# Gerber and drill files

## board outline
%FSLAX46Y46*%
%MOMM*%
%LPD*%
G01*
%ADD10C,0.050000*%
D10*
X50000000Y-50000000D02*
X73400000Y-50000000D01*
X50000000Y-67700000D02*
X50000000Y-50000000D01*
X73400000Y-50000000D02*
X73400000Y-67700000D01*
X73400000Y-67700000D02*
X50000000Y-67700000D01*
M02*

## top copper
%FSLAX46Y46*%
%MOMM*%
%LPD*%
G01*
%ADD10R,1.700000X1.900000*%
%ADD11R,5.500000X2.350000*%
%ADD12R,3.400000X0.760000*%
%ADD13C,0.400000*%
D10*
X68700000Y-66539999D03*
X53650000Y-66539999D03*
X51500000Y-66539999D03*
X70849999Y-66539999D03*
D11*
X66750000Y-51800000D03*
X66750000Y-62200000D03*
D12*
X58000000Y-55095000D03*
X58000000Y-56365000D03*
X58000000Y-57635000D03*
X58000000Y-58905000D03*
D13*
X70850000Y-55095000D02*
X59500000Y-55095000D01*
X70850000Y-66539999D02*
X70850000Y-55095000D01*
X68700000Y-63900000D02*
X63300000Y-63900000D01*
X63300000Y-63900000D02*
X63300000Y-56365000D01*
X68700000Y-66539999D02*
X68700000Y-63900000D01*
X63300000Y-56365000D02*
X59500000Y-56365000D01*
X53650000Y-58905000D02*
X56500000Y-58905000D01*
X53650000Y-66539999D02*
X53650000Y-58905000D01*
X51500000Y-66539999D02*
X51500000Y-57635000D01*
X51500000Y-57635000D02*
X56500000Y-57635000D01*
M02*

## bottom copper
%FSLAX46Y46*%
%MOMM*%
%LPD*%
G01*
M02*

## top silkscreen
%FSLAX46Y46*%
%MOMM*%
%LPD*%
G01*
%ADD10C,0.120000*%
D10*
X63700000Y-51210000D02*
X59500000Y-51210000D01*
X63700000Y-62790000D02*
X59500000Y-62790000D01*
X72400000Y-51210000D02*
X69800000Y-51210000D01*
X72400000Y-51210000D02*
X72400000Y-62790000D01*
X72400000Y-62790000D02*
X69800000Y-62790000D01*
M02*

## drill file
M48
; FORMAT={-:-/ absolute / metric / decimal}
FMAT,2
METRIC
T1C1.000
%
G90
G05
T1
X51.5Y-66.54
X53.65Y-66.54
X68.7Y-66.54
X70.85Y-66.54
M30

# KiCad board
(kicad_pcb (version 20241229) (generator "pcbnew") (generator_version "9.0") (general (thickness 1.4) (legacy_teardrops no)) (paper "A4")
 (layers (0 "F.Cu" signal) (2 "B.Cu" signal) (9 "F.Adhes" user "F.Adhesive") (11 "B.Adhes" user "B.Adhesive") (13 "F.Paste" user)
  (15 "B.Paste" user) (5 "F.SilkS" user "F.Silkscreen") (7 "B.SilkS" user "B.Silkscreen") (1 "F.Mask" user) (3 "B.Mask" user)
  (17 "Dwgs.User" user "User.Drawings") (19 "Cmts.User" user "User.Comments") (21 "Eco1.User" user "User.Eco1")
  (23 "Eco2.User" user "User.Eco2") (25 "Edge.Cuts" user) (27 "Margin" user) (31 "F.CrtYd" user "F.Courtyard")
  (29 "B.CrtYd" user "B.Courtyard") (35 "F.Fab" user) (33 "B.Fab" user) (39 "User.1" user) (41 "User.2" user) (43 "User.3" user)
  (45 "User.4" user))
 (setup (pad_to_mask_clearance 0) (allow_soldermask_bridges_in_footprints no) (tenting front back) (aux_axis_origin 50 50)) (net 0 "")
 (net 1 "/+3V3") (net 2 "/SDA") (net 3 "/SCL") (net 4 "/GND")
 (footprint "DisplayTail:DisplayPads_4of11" (layer "F.Cu") (at 51.5 66.539999)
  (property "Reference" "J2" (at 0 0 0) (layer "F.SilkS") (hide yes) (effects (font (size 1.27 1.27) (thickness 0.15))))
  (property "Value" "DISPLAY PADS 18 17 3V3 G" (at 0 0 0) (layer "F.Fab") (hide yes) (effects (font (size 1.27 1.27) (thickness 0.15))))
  (pad "3V3" thru_hole rect (at 17.2 0) (size 1.7 1.9) (drill 1) (layers "*.Cu" "*.Mask") (remove_unused_layers yes) (keep_end_layers no)
   (zone_layer_connections) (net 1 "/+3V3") (thermal_bridge_angle 45))
  (pad "17" thru_hole rect (at 2.15 0) (size 1.7 1.9) (drill 1) (layers "*.Cu" "*.Mask") (remove_unused_layers yes) (keep_end_layers no)
   (zone_layer_connections) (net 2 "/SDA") (thermal_bridge_angle 45))
  (pad "18" thru_hole rect (at 0 0) (size 1.7 1.9) (drill 1) (layers "*.Cu" "*.Mask") (remove_unused_layers yes) (keep_end_layers no)
   (zone_layer_connections) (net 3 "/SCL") (thermal_bridge_angle 45))
  (pad "G" thru_hole rect (at 19.349999 0) (size 1.7 1.9) (drill 1) (layers "*.Cu" "*.Mask") (remove_unused_layers yes) (keep_end_layers no)
   (zone_layer_connections) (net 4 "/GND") (thermal_bridge_angle 45)))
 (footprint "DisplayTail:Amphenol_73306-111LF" (layer "F.Cu") (at 72.4 57 -90)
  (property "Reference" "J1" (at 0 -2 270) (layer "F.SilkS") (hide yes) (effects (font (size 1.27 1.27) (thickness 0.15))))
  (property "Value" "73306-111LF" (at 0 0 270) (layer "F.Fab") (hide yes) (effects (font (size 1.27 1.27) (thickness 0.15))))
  (fp_line (start -5.79 8.7) (end -5.79 12.9) (stroke (width 0.12) (type default)) (layer "F.SilkS"))
  (fp_line (start 5.79 8.7) (end 5.79 12.9) (stroke (width 0.12) (type default)) (layer "F.SilkS"))
  (fp_line (start -5.79 0) (end -5.79 2.6) (stroke (width 0.12) (type default)) (layer "F.SilkS"))
  (fp_line (start -5.79 0) (end 5.79 0) (stroke (width 0.12) (type default)) (layer "F.SilkS"))
  (fp_line (start 5.79 0) (end 5.79 2.6) (stroke (width 0.12) (type default)) (layer "F.SilkS"))
  (pad "" smd rect (at -5.2 5.65 270) (size 2.35 5.5) (layers "F.Cu" "F.Mask" "F.Paste") (thermal_bridge_angle 45))
  (pad "" smd rect (at 5.2 5.65 270) (size 2.35 5.5) (layers "F.Cu" "F.Mask" "F.Paste") (thermal_bridge_angle 45))
  (pad "1" smd rect (at -1.905 14.4 270) (size 0.76 3.4) (layers "F.Cu" "F.Mask" "F.Paste") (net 4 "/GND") (thermal_bridge_angle 45))
  (pad "2" smd rect (at -0.635 14.4 270) (size 0.76 3.4) (layers "F.Cu" "F.Mask" "F.Paste") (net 1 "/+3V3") (thermal_bridge_angle 45))
  (pad "3" smd rect (at 0.635 14.4 270) (size 0.76 3.4) (layers "F.Cu" "F.Mask" "F.Paste") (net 3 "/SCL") (thermal_bridge_angle 45))
  (pad "4" smd rect (at 1.905 14.4 270) (size 0.76 3.4) (layers "F.Cu" "F.Mask" "F.Paste") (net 2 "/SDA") (thermal_bridge_angle 45)))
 (gr_line (start 50 50) (end 73.4 50) (stroke (width 0.05) (type default)) (layer "Edge.Cuts"))
 (gr_line (start 50 67.7) (end 50 50) (stroke (width 0.05) (type default)) (layer "Edge.Cuts"))
 (gr_line (start 73.4 50) (end 73.4 67.7) (stroke (width 0.05) (type default)) (layer "Edge.Cuts"))
 (gr_line (start 73.4 67.7) (end 50 67.7) (stroke (width 0.05) (type default)) (layer "Edge.Cuts"))
 (segment (start 70.85 55.095) (end 59.5 55.095) (width 0.4) (layer "F.Cu") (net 4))
 (segment (start 70.85 66.539999) (end 70.85 55.095) (width 0.4) (layer "F.Cu") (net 4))
 (segment (start 68.7 63.9) (end 63.3 63.9) (width 0.4) (layer "F.Cu") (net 1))
 (segment (start 63.3 63.9) (end 63.3 56.365) (width 0.4) (layer "F.Cu") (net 1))
 (segment (start 68.7 66.539999) (end 68.7 63.9) (width 0.4) (layer "F.Cu") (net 1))
 (segment (start 63.3 56.365) (end 59.5 56.365) (width 0.4) (layer "F.Cu") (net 1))
 (segment (start 53.65 58.905) (end 56.5 58.905) (width 0.4) (layer "F.Cu") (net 2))
 (segment (start 53.65 66.539999) (end 53.65 58.905) (width 0.4) (layer "F.Cu") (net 2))
 (segment (start 51.5 66.539999) (end 51.5 57.635) (width 0.4) (layer "F.Cu") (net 3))
 (segment (start 51.5 57.635) (end 56.5 57.635) (width 0.4) (layer "F.Cu") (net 3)))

